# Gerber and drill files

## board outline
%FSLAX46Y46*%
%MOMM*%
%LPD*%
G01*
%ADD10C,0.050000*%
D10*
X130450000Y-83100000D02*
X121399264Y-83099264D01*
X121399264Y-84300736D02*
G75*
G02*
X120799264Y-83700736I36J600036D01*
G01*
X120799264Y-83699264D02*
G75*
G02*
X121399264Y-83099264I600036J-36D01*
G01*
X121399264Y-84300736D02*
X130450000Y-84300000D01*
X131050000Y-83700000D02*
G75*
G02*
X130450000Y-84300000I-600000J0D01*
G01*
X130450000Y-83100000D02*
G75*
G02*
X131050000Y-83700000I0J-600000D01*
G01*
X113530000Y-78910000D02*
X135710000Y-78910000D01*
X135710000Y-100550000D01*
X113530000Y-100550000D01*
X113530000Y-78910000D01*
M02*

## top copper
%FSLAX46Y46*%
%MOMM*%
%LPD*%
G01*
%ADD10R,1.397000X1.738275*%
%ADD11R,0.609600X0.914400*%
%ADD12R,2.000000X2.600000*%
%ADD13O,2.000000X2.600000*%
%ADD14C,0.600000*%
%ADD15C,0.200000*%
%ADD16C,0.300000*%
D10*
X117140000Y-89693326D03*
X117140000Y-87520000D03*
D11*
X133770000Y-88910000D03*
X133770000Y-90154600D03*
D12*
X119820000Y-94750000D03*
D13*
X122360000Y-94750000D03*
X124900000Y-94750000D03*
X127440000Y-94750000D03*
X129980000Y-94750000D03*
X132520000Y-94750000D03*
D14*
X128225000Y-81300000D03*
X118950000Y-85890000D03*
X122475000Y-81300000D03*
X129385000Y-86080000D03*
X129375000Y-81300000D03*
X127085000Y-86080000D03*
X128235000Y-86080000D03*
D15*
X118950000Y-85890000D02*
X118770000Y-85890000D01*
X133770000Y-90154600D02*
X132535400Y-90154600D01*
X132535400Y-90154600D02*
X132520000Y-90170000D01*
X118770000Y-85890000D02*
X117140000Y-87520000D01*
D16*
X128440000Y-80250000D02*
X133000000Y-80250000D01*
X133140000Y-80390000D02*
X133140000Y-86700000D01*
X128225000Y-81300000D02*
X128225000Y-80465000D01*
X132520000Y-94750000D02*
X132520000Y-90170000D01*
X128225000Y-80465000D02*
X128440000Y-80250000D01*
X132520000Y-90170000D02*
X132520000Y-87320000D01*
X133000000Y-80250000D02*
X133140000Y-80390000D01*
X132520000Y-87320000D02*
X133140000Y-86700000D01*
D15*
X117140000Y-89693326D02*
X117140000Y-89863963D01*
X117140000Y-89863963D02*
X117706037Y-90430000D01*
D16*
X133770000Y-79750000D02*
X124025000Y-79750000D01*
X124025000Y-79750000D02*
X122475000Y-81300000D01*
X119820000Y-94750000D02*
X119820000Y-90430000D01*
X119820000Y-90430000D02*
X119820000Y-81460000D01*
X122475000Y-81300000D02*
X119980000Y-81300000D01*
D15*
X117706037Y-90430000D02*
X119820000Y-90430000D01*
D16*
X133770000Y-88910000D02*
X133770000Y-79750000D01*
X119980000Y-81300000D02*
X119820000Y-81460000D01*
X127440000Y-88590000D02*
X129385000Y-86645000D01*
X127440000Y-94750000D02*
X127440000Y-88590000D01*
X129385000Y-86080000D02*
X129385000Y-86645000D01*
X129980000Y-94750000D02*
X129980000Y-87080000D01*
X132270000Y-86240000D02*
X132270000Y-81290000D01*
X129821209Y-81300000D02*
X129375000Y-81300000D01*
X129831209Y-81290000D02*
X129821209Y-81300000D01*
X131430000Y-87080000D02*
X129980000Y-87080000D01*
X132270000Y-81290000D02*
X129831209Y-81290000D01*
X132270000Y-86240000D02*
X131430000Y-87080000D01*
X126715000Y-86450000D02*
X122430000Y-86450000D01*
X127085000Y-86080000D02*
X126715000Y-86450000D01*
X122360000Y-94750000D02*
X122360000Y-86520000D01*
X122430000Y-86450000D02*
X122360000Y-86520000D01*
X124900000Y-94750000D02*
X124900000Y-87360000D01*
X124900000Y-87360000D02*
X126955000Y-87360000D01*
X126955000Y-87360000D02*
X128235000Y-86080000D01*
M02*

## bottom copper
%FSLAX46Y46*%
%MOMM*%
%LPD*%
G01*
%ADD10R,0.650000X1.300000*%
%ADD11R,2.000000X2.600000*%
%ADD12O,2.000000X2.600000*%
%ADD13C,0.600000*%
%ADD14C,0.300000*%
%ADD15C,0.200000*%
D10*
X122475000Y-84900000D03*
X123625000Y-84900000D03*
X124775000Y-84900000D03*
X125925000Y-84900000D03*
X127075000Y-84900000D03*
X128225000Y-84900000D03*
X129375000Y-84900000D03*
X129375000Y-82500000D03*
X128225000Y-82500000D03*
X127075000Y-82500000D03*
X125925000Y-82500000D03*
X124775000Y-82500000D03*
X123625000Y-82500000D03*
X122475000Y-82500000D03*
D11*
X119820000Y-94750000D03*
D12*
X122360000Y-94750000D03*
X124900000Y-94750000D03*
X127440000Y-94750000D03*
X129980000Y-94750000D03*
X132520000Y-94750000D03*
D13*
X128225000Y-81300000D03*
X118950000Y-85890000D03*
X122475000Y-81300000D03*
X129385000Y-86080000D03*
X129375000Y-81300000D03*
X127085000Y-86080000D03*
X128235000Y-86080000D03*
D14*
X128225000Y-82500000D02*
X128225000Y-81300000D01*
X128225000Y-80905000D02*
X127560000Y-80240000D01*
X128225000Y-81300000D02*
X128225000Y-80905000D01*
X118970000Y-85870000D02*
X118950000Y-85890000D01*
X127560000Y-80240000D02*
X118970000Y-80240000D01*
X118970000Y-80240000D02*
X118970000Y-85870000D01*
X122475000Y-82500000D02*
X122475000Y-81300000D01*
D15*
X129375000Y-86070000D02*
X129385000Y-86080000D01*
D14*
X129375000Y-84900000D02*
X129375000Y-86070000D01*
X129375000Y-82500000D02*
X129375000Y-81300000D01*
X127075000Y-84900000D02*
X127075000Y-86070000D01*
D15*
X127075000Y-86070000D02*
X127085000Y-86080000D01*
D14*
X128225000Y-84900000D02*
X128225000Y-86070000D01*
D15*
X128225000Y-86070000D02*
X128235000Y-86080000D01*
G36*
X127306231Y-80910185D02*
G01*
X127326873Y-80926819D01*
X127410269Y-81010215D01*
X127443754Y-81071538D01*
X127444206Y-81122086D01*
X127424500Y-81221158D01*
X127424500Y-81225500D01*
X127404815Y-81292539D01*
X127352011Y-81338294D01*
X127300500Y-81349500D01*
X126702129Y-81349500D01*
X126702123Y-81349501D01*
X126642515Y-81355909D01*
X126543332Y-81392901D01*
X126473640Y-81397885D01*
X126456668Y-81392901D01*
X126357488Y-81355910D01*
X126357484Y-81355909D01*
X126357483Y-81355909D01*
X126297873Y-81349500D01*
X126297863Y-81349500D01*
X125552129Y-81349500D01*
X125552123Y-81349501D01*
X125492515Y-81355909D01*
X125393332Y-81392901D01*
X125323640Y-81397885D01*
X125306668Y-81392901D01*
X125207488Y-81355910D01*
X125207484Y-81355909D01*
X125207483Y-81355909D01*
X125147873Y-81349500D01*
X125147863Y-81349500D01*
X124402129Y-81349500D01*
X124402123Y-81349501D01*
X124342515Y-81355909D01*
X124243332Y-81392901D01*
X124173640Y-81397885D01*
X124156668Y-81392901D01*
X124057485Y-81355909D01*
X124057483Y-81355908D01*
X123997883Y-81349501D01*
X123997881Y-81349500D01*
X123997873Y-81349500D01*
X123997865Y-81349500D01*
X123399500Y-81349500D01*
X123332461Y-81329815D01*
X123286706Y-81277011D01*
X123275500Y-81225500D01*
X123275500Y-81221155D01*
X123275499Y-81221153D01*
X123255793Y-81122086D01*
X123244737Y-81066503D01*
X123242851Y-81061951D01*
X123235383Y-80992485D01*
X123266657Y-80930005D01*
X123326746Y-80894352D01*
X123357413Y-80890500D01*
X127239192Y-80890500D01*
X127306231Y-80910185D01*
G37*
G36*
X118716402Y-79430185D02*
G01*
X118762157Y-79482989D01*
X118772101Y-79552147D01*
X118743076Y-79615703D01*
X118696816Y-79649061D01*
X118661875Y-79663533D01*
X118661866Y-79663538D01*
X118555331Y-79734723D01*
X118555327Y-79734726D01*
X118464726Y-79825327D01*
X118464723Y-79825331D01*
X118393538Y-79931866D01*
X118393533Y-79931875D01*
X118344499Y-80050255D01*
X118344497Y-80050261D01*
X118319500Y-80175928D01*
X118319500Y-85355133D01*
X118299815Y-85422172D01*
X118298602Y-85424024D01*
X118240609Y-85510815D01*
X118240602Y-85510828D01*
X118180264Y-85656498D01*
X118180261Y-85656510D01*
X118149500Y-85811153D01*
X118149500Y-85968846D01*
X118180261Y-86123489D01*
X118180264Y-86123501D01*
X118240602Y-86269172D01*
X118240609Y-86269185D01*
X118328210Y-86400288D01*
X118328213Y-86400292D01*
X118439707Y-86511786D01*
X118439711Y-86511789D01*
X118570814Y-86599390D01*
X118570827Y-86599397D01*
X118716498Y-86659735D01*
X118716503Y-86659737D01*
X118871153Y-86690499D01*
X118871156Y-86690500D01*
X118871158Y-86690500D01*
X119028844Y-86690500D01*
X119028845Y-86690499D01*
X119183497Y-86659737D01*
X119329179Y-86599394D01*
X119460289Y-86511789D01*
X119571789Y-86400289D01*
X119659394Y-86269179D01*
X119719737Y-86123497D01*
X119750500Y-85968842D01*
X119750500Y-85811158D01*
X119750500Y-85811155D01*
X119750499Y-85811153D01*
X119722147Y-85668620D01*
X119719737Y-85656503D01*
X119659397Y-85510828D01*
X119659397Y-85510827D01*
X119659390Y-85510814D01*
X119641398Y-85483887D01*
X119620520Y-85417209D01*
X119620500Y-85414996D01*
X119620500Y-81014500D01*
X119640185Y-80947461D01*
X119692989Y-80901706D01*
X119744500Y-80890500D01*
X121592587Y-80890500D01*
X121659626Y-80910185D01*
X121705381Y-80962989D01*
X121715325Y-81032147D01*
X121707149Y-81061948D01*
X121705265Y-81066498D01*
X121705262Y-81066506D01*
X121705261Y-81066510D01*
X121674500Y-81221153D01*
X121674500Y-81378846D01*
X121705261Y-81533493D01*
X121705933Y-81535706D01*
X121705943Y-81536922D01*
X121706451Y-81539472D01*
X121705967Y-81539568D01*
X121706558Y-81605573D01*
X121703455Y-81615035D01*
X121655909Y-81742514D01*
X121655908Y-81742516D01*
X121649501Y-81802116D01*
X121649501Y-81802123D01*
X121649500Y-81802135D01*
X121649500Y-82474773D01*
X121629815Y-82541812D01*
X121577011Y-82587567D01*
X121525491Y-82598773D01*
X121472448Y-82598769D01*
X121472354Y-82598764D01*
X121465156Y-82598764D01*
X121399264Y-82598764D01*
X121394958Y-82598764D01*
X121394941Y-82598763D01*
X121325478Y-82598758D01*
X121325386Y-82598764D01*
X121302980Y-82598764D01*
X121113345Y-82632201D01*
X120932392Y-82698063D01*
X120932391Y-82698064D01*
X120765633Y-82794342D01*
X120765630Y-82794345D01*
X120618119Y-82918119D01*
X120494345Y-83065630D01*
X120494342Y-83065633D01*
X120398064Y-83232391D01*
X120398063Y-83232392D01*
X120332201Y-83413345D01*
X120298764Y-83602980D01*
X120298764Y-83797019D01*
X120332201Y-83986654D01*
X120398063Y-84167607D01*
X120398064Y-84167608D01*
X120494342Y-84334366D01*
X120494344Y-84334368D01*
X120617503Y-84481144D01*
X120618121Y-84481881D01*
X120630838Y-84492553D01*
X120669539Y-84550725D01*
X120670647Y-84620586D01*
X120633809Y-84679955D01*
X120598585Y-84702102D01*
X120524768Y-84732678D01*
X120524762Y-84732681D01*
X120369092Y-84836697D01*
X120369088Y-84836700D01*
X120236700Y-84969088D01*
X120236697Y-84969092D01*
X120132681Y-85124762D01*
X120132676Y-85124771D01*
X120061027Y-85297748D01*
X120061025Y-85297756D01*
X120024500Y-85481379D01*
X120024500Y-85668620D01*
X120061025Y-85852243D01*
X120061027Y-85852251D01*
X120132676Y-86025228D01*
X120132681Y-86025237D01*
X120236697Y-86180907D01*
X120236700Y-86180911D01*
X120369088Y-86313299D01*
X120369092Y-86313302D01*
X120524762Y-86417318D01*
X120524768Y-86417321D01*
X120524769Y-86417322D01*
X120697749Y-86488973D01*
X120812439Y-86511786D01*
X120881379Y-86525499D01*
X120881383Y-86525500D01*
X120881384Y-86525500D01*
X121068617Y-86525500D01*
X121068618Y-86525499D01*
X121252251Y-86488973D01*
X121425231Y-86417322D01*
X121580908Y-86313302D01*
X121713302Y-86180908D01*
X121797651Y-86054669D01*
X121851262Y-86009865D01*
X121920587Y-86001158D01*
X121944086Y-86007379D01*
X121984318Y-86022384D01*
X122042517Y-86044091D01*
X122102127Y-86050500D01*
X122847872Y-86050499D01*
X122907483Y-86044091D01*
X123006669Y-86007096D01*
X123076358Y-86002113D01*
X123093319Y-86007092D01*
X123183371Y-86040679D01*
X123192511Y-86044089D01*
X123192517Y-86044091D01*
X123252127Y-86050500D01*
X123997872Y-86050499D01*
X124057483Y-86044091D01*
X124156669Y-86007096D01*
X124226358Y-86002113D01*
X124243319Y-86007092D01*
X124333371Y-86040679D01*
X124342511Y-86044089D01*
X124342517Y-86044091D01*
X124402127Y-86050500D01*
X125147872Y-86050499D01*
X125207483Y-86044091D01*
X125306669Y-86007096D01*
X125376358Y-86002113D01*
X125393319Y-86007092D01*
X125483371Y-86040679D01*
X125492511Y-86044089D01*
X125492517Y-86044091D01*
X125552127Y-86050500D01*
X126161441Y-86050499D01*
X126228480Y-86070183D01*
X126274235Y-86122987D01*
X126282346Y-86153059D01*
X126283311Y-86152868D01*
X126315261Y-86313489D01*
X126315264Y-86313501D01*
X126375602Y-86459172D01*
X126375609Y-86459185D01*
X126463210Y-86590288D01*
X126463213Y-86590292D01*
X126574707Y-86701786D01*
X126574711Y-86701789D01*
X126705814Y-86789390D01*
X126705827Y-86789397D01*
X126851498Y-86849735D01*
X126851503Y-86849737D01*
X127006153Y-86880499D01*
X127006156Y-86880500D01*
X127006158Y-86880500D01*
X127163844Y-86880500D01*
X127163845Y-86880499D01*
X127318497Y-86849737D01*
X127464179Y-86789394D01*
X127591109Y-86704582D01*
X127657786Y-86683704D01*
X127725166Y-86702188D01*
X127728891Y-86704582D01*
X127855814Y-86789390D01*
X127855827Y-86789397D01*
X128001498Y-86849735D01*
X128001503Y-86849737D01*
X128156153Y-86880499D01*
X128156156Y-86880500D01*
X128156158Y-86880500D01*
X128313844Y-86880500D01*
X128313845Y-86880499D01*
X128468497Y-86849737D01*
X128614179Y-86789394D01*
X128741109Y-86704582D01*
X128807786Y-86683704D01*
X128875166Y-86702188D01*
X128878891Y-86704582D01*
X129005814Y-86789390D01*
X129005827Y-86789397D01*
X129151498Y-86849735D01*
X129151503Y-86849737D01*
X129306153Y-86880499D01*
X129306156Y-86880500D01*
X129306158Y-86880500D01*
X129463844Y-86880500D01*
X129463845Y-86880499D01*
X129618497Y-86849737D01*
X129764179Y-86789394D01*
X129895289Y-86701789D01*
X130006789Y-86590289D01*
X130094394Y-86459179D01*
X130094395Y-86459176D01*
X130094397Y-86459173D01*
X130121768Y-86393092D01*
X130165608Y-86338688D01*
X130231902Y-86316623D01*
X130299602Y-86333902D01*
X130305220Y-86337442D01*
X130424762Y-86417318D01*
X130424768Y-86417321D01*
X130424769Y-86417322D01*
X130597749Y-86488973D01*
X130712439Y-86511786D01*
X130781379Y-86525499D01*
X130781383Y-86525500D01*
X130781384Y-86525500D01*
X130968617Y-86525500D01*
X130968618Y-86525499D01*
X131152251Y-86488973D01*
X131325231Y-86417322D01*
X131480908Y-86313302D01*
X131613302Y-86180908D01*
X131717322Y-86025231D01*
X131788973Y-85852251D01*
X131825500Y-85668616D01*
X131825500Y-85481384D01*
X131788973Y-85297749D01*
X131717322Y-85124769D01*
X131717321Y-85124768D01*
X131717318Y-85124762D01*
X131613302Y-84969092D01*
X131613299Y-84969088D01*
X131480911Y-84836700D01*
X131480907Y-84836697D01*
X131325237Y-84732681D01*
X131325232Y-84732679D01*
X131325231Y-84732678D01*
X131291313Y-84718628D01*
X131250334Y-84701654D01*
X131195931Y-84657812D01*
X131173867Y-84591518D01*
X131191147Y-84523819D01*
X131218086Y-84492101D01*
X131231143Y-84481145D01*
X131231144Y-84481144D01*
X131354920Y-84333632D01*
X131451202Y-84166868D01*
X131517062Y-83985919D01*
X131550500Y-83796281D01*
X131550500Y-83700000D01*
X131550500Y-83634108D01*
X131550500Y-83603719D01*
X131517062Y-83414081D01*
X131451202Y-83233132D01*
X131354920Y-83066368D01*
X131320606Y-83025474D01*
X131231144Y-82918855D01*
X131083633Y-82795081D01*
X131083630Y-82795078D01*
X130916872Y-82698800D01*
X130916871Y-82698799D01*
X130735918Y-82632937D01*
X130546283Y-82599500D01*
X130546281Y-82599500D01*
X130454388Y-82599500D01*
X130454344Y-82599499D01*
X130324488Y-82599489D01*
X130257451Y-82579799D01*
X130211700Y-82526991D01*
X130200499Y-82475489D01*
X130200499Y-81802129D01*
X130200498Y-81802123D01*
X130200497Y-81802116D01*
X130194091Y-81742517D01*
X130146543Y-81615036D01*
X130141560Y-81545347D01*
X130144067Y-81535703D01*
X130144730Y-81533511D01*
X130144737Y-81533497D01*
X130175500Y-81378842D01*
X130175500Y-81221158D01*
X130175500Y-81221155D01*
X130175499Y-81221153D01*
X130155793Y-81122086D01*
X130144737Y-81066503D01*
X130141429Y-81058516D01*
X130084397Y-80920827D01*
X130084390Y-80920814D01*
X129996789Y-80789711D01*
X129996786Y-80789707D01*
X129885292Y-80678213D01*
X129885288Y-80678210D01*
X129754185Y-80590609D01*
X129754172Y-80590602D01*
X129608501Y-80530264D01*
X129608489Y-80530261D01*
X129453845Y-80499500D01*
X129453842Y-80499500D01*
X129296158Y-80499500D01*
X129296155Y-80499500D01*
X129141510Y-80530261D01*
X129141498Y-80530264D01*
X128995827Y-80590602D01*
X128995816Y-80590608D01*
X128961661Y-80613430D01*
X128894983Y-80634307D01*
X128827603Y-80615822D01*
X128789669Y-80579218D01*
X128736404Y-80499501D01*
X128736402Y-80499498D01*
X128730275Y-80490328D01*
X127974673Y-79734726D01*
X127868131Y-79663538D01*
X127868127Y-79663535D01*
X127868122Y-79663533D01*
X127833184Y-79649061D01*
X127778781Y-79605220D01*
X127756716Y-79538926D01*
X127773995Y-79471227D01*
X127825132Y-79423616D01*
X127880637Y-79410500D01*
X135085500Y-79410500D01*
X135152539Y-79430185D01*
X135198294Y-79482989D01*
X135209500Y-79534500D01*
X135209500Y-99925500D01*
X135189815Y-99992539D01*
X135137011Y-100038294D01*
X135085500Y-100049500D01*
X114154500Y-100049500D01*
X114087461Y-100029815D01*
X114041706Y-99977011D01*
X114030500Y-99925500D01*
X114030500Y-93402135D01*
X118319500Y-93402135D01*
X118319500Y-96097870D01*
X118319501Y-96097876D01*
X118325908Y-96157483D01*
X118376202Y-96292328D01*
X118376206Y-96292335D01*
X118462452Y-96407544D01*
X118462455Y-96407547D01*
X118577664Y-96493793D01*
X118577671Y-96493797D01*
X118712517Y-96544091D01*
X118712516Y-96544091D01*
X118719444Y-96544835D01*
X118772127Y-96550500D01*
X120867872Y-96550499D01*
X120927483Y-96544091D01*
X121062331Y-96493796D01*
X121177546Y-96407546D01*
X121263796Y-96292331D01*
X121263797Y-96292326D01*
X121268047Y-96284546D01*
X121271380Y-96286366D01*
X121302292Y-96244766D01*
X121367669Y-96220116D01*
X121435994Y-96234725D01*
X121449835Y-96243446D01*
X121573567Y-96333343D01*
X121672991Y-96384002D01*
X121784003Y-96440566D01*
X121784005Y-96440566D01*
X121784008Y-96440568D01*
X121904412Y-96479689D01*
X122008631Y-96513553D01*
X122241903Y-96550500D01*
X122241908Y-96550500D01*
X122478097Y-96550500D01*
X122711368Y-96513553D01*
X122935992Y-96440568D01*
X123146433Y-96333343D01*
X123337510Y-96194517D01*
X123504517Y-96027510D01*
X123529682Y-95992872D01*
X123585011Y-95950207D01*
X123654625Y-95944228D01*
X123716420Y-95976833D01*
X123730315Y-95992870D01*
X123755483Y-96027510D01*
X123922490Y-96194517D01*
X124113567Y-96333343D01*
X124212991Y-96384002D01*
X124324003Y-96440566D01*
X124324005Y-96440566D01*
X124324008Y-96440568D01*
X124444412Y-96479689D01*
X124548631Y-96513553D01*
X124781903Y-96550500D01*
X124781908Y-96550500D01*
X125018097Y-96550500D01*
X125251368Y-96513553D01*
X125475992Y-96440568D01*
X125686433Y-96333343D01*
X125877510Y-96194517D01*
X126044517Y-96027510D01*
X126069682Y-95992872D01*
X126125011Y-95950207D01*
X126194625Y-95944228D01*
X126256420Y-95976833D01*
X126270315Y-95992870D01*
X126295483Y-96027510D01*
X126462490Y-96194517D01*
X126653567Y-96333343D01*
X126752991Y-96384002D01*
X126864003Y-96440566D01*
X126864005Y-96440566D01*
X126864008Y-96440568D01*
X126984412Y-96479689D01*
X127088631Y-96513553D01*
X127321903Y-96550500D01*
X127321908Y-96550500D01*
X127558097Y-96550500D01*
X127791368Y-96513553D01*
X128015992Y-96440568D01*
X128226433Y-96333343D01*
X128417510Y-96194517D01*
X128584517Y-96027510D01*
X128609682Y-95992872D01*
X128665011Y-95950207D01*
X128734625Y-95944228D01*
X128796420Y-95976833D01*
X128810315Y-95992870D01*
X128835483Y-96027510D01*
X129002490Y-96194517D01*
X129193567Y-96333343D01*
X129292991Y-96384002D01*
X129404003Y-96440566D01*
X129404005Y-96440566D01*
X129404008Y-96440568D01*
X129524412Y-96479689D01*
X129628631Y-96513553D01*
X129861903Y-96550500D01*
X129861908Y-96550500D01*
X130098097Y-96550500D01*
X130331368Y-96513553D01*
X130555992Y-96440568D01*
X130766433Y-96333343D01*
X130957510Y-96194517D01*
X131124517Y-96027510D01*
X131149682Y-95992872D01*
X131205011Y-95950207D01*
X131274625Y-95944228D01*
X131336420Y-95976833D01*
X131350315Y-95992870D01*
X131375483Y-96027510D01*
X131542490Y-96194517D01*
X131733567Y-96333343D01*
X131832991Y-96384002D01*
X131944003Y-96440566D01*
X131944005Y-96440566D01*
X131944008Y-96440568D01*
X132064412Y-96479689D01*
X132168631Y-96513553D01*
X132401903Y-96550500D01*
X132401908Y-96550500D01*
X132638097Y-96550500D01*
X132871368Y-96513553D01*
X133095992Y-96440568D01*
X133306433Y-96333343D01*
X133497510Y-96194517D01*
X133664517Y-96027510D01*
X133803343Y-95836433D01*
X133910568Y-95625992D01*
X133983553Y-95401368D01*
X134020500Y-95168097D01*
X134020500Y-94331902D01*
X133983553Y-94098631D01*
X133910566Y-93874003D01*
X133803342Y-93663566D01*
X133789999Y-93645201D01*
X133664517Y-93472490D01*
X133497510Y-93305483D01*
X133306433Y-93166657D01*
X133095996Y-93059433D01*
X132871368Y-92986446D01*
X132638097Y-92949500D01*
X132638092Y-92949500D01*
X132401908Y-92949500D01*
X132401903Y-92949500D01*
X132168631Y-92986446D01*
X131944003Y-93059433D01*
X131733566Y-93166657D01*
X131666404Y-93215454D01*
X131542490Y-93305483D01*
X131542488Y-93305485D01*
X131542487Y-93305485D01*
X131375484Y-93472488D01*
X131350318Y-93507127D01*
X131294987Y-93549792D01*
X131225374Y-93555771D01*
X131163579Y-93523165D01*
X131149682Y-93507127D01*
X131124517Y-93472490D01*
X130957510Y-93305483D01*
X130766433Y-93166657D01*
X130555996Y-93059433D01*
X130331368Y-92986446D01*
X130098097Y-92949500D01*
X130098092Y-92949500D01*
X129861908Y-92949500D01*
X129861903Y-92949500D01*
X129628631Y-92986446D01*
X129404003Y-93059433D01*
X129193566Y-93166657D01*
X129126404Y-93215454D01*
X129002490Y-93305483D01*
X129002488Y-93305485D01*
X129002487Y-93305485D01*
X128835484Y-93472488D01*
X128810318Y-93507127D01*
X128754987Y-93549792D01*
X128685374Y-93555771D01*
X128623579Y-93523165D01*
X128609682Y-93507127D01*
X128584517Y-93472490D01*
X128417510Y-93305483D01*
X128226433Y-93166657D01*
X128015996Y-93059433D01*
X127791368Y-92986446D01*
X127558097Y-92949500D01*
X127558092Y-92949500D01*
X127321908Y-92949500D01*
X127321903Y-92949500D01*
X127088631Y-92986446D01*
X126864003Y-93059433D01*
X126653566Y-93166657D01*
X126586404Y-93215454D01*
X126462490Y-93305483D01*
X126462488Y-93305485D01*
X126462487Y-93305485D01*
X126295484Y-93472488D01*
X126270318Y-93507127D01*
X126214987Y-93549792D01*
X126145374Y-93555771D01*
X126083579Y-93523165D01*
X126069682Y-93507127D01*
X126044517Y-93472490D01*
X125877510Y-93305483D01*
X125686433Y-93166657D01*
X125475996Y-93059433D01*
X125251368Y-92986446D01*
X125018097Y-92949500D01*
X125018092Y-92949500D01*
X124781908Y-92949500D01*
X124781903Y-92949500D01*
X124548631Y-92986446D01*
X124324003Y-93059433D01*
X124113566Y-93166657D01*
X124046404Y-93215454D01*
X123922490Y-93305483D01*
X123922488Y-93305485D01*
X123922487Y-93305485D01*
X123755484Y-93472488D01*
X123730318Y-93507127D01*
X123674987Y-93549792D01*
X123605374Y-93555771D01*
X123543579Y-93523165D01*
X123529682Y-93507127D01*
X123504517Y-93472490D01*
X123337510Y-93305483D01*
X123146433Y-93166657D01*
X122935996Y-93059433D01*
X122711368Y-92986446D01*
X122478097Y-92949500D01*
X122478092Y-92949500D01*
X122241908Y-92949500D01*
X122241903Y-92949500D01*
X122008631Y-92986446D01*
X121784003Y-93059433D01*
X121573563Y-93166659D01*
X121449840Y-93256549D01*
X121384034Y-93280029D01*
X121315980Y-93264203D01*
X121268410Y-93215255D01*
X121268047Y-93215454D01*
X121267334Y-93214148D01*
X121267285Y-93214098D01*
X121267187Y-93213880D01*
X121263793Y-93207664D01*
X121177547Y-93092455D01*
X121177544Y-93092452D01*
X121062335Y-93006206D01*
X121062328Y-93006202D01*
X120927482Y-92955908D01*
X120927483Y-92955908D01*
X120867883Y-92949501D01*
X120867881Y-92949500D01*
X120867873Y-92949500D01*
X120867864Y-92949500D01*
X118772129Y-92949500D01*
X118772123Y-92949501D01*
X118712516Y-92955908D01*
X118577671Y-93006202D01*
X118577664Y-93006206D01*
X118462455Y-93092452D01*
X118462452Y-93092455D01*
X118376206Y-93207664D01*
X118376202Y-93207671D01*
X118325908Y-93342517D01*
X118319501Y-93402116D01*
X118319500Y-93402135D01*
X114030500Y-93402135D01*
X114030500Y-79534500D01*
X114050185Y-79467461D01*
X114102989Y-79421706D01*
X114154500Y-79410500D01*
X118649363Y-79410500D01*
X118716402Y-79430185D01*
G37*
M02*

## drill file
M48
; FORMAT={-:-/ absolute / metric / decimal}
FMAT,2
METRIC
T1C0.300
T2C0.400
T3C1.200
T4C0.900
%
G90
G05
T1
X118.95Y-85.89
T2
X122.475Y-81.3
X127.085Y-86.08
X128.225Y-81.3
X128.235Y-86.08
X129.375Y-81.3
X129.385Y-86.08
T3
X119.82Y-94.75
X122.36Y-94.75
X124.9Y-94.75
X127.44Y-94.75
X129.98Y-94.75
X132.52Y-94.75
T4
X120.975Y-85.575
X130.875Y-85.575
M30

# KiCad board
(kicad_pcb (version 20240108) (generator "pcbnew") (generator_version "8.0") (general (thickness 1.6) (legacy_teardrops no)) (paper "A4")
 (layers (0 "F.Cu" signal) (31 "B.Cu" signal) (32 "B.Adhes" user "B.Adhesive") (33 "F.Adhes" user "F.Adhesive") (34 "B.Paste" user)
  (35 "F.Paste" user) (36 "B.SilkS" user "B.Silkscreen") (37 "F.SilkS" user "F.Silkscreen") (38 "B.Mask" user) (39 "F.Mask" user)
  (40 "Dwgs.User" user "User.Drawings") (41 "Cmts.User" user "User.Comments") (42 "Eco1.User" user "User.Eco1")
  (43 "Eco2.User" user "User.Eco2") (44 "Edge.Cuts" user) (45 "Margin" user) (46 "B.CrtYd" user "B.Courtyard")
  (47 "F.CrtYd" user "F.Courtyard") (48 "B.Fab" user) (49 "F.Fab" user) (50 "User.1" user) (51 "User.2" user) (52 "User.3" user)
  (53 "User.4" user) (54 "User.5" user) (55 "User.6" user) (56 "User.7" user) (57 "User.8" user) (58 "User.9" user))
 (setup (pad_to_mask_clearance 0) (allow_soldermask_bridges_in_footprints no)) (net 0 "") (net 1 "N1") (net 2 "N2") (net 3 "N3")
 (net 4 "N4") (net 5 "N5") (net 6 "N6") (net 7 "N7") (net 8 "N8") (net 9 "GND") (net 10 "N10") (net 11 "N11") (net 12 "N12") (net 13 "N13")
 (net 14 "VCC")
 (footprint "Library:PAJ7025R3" (layer "F.Cu") (at 125.925 83.7)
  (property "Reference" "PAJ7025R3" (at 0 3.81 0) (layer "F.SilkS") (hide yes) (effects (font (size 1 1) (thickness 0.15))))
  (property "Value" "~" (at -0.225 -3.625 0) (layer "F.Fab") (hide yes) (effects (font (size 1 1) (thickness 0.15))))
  (pad "" np_thru_hole oval (at -4.95 1.875) (size 0.9 0.9) (drill 0.9) (layers "F&B.Cu"))
  (pad "" np_thru_hole oval (at 4.95 1.875) (size 0.9 0.9) (drill 0.9) (layers "*.Cu"))
  (pad "1" smd rect (at -3.45 1.2) (size 0.65 1.3) (layers "B.Cu" "B.Paste" "B.Mask") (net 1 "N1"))
  (pad "2" smd rect (at -2.3 1.2) (size 0.65 1.3) (layers "B.Cu" "B.Paste" "B.Mask") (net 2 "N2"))
  (pad "3" smd rect (at -1.15 1.2) (size 0.65 1.3) (layers "B.Cu" "B.Paste" "B.Mask") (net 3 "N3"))
  (pad "4" smd rect (at 0 1.2) (size 0.65 1.3) (layers "B.Cu" "B.Paste" "B.Mask") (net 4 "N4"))
  (pad "5" smd rect (at 1.15 1.2) (size 0.65 1.3) (layers "B.Cu" "B.Paste" "B.Mask") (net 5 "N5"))
  (pad "6" smd rect (at 2.3 1.2) (size 0.65 1.3) (layers "B.Cu" "B.Paste" "B.Mask") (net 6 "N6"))
  (pad "7" smd rect (at 3.45 1.2) (size 0.65 1.3) (layers "B.Cu" "B.Paste" "B.Mask") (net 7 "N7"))
  (pad "8" smd rect (at 3.45 -1.2) (size 0.65 1.3) (layers "B.Cu" "B.Paste" "B.Mask") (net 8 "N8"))
  (pad "9" smd rect (at 2.3 -1.2) (size 0.65 1.3) (layers "B.Cu" "B.Paste" "B.Mask") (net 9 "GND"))
  (pad "10" smd rect (at 1.15 -1.2) (size 0.65 1.3) (layers "B.Cu" "B.Paste" "B.Mask") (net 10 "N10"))
  (pad "11" smd rect (at 0 -1.2) (size 0.65 1.3) (layers "B.Cu" "B.Paste" "B.Mask") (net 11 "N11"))
  (pad "12" smd rect (at -1.15 -1.2) (size 0.65 1.3) (layers "B.Cu" "B.Paste" "B.Mask") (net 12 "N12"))
  (pad "13" smd rect (at -2.3 -1.2) (size 0.65 1.3) (layers "B.Cu" "B.Paste" "B.Mask") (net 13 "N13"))
  (pad "14" smd rect (at -3.45 -1.2) (size 0.65 1.3) (layers "B.Cu" "B.Paste" "B.Mask") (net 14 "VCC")))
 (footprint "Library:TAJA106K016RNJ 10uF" (layer "F.Cu") (at 117.14 88.606663 90)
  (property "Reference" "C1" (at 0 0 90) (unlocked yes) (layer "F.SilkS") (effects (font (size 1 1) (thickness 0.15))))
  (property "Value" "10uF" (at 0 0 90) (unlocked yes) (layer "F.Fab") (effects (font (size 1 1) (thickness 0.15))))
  (pad "1" smd rect (at -1.086663 0 180) (size 1.397 1.738275) (layers "F.Cu" "F.Paste" "F.Mask") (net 14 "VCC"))
  (pad "2" smd rect (at 1.086663 0 180) (size 1.397 1.738275) (layers "F.Cu" "F.Paste" "F.Mask") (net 9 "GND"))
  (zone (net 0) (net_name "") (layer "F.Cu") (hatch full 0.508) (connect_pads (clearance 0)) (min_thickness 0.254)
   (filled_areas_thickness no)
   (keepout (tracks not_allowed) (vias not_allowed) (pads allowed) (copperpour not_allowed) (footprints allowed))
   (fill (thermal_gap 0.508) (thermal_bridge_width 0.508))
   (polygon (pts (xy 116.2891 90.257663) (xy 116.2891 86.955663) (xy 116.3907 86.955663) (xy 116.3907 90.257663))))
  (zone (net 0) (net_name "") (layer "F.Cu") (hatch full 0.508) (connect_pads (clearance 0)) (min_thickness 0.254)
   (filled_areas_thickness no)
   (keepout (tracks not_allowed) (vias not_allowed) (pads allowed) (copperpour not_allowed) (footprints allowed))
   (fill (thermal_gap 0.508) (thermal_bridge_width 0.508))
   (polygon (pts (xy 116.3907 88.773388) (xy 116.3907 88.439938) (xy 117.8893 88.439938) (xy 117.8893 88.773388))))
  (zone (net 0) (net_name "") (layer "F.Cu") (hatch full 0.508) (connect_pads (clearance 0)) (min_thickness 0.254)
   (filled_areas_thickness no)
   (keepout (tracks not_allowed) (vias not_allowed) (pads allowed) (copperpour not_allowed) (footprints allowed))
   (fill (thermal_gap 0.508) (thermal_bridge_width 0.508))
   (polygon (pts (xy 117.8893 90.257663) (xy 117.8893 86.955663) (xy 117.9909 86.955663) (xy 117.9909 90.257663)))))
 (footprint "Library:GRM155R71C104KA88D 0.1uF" (layer "F.Cu") (at 133.77 89.5323 -90)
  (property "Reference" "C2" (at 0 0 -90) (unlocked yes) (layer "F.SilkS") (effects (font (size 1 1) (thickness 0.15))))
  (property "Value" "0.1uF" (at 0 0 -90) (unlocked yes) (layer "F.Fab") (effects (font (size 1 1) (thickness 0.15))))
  (pad "1" smd rect (at -0.6223 0 270) (size 0.9144 0.6096) (layers "F.Cu" "F.Paste" "F.Mask") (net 14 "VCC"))
  (pad "2" smd rect (at 0.6223 0 270) (size 0.9144 0.6096) (layers "F.Cu" "F.Paste" "F.Mask") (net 9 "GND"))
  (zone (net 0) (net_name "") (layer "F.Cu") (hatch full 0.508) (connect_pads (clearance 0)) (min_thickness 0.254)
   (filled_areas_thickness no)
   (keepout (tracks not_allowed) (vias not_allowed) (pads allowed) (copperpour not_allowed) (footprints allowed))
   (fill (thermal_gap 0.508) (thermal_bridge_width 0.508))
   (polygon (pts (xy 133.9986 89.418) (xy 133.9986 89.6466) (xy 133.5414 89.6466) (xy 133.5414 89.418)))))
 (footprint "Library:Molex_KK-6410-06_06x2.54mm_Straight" (layer "F.Cu") (at 119.82 94.75)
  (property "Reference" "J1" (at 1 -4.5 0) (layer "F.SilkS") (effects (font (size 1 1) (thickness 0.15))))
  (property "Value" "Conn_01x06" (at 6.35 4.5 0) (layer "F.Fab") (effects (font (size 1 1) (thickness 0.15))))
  (pad "1" thru_hole rect (at 0 0) (size 2 2.6) (drill 1.2) (layers "*.Cu" "*.Mask") (remove_unused_layers yes) (keep_end_layers yes)
   (zone_layer_connections) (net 14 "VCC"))
  (pad "2" thru_hole oval (at 2.54 0) (size 2 2.6) (drill 1.2) (layers "*.Cu" "*.Mask") (remove_unused_layers yes) (keep_end_layers yes)
   (zone_layer_connections) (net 5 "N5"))
  (pad "3" thru_hole oval (at 5.08 0) (size 2 2.6) (drill 1.2) (layers "*.Cu" "*.Mask") (remove_unused_layers yes) (keep_end_layers yes)
   (zone_layer_connections) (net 6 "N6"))
  (pad "4" thru_hole oval (at 7.62 0) (size 2 2.6) (drill 1.2) (layers "*.Cu" "*.Mask") (remove_unused_layers yes) (keep_end_layers yes)
   (zone_layer_connections) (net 7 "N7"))
  (pad "5" thru_hole oval (at 10.16 0) (size 2 2.6) (drill 1.2) (layers "*.Cu" "*.Mask") (remove_unused_layers yes) (keep_end_layers yes)
   (zone_layer_connections) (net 8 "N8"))
  (pad "6" thru_hole oval (at 12.7 0) (size 2 2.6) (drill 1.2) (layers "*.Cu" "*.Mask") (remove_unused_layers yes) (keep_end_layers yes)
   (zone_layer_connections) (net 9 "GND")))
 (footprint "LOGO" (layer "F.Cu") (at 116.57 83.13)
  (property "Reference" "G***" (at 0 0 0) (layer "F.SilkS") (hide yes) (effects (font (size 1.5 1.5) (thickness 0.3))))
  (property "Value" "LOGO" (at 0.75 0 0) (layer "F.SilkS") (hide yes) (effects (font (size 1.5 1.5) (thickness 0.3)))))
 (gr_line (start 130.45 83.1) (end 121.399264 83.099264) (stroke (width 0.05) (type default)) (layer "Edge.Cuts"))
 (gr_arc (start 121.399264 84.300736) (mid 120.975 84.125) (end 120.799264 83.700736) (stroke (width 0.05) (type default))
  (layer "Edge.Cuts"))
 (gr_arc (start 120.799264 83.699264) (mid 120.975 83.275) (end 121.399264 83.099264) (stroke (width 0.05) (type default))
  (layer "Edge.Cuts"))
 (gr_line (start 121.399264 84.300736) (end 130.45 84.3) (stroke (width 0.05) (type default)) (layer "Edge.Cuts"))
 (gr_arc (start 131.05 83.7) (mid 130.874264 84.124264) (end 130.45 84.3) (stroke (width 0.05) (type default)) (layer "Edge.Cuts"))
 (gr_arc (start 130.45 83.1) (mid 130.874264 83.275736) (end 131.05 83.7) (stroke (width 0.05) (type default)) (layer "Edge.Cuts"))
 (gr_rect (start 113.53 78.91) (end 135.71 100.55) (stroke (width 0.05) (type default)) (fill none) (layer "Edge.Cuts"))
 (segment (start 118.95 85.89) (end 118.77 85.89) (width 0.2) (layer "F.Cu") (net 9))
 (segment (start 133.77 90.1546) (end 132.5354 90.1546) (width 0.2) (layer "F.Cu") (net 9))
 (segment (start 132.5354 90.1546) (end 132.52 90.17) (width 0.2) (layer "F.Cu") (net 9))
 (segment (start 118.77 85.89) (end 117.14 87.52) (width 0.2) (layer "F.Cu") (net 9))
 (segment (start 128.44 80.25) (end 133 80.25) (width 0.3) (layer "F.Cu") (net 9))
 (segment (start 133.14 80.39) (end 133.14 86.7) (width 0.3) (layer "F.Cu") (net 9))
 (segment (start 128.225 81.3) (end 128.225 80.465) (width 0.3) (layer "F.Cu") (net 9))
 (segment (start 132.52 94.75) (end 132.52 90.17) (width 0.3) (layer "F.Cu") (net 9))
 (segment (start 128.225 80.465) (end 128.44 80.25) (width 0.3) (layer "F.Cu") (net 9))
 (segment (start 132.52 90.17) (end 132.52 87.32) (width 0.3) (layer "F.Cu") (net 9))
 (segment (start 133 80.25) (end 133.14 80.39) (width 0.3) (layer "F.Cu") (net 9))
 (segment (start 132.52 87.32) (end 133.14 86.7) (width 0.3) (layer "F.Cu") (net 9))
 (via (at 128.225 81.3) (size 0.6) (drill 0.4) (layers "F.Cu" "B.Cu") (remove_unused_layers yes) (keep_end_layers yes) (free yes)
  (zone_layer_connections) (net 9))
 (via (at 118.95 85.89) (size 0.6) (drill 0.3) (layers "F.Cu" "B.Cu") (remove_unused_layers yes) (keep_end_layers yes)
  (zone_layer_connections) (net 9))
 (segment (start 128.225 82.5) (end 128.225 81.3) (width 0.3) (layer "B.Cu") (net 9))
 (segment (start 128.225 80.905) (end 127.56 80.24) (width 0.3) (layer "B.Cu") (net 9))
 (segment (start 128.225 81.3) (end 128.225 80.905) (width 0.3) (layer "B.Cu") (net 9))
 (segment (start 118.97 85.87) (end 118.95 85.89) (width 0.3) (layer "B.Cu") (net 9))
 (segment (start 127.56 80.24) (end 118.97 80.24) (width 0.3) (layer "B.Cu") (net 9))
 (segment (start 118.97 80.24) (end 118.97 85.87) (width 0.3) (layer "B.Cu") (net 9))
 (segment (start 117.14 89.693326) (end 117.14 89.863963) (width 0.2) (layer "F.Cu") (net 14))
 (segment (start 117.14 89.863963) (end 117.706037 90.43) (width 0.2) (layer "F.Cu") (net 14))
 (segment (start 133.77 79.75) (end 124.025 79.75) (width 0.3) (layer "F.Cu") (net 14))
 (segment (start 124.025 79.75) (end 122.475 81.3) (width 0.3) (layer "F.Cu") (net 14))
 (segment (start 119.82 94.75) (end 119.82 90.43) (width 0.3) (layer "F.Cu") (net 14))
 (segment (start 119.82 90.43) (end 119.82 81.46) (width 0.3) (layer "F.Cu") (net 14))
 (segment (start 122.475 81.3) (end 119.98 81.3) (width 0.3) (layer "F.Cu") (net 14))
 (segment (start 117.706037 90.43) (end 119.82 90.43) (width 0.2) (layer "F.Cu") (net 14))
 (segment (start 133.77 88.91) (end 133.77 79.75) (width 0.3) (layer "F.Cu") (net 14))
 (segment (start 119.98 81.3) (end 119.82 81.46) (width 0.3) (layer "F.Cu") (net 14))
 (via (at 122.475 81.3) (size 0.6) (drill 0.4) (layers "F.Cu" "B.Cu") (remove_unused_layers yes) (keep_end_layers yes) (free yes)
  (zone_layer_connections) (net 14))
 (segment (start 122.475 82.5) (end 122.475 81.3) (width 0.3) (layer "B.Cu") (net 14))
 (segment (start 127.44 88.59) (end 129.385 86.645) (width 0.3) (layer "F.Cu") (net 7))
 (segment (start 127.44 94.75) (end 127.44 88.59) (width 0.3) (layer "F.Cu") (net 7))
 (segment (start 129.385 86.08) (end 129.385 86.645) (width 0.3) (layer "F.Cu") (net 7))
 (via (at 129.385 86.08) (size 0.6) (drill 0.4) (layers "F.Cu" "B.Cu") (remove_unused_layers yes) (keep_end_layers yes) (free yes)
  (zone_layer_connections) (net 7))
 (segment (start 129.375 86.07) (end 129.385 86.08) (width 0.2) (layer "B.Cu") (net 7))
 (segment (start 129.375 84.9) (end 129.375 86.07) (width 0.3) (layer "B.Cu") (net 7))
 (segment (start 129.98 94.75) (end 129.98 87.08) (width 0.3) (layer "F.Cu") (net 8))
 (segment (start 132.27 86.24) (end 132.27 81.29) (width 0.3) (layer "F.Cu") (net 8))
 (segment (start 129.821209 81.3) (end 129.375 81.3) (width 0.3) (layer "F.Cu") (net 8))
 (segment (start 129.831209 81.29) (end 129.821209 81.3) (width 0.3) (layer "F.Cu") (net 8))
 (segment (start 131.43 87.08) (end 129.98 87.08) (width 0.3) (layer "F.Cu") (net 8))
 (segment (start 132.27 81.29) (end 129.831209 81.29) (width 0.3) (layer "F.Cu") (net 8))
 (segment (start 132.27 86.24) (end 131.43 87.08) (width 0.3) (layer "F.Cu") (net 8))
 (via (at 129.375 81.3) (size 0.6) (drill 0.4) (layers "F.Cu" "B.Cu") (remove_unused_layers yes) (keep_end_layers yes) (free yes)
  (zone_layer_connections) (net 8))
 (segment (start 129.375 82.5) (end 129.375 81.3) (width 0.3) (layer "B.Cu") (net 8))
 (segment (start 126.715 86.45) (end 122.43 86.45) (width 0.3) (layer "F.Cu") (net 5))
 (segment (start 127.085 86.08) (end 126.715 86.45) (width 0.3) (layer "F.Cu") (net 5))
 (segment (start 122.36 94.75) (end 122.36 86.52) (width 0.3) (layer "F.Cu") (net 5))
 (segment (start 122.43 86.45) (end 122.36 86.52) (width 0.3) (layer "F.Cu") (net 5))
 (via (at 127.085 86.08) (size 0.6) (drill 0.4) (layers "F.Cu" "B.Cu") (remove_unused_layers yes) (keep_end_layers yes) (free yes)
  (zone_layer_connections) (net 5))
 (segment (start 127.075 84.9) (end 127.075 86.07) (width 0.3) (layer "B.Cu") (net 5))
 (segment (start 127.075 86.07) (end 127.085 86.08) (width 0.2) (layer "B.Cu") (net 5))
 (segment (start 124.9 94.75) (end 124.9 87.36) (width 0.3) (layer "F.Cu") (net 6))
 (segment (start 124.9 87.36) (end 126.955 87.36) (width 0.3) (layer "F.Cu") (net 6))
 (segment (start 126.955 87.36) (end 128.235 86.08) (width 0.3) (layer "F.Cu") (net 6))
 (via (at 128.235 86.08) (size 0.6) (drill 0.4) (layers "F.Cu" "B.Cu") (remove_unused_layers yes) (keep_end_layers yes) (free yes)
  (zone_layer_connections) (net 6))
 (segment (start 128.225 84.9) (end 128.225 86.07) (width 0.3) (layer "B.Cu") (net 6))
 (segment (start 128.225 86.07) (end 128.235 86.08) (width 0.2) (layer "B.Cu") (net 6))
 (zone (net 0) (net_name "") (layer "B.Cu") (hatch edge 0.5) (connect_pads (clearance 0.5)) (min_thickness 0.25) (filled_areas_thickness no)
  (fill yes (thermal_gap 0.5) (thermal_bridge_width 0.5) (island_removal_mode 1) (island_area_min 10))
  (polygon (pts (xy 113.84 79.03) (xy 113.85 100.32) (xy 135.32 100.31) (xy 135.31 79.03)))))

